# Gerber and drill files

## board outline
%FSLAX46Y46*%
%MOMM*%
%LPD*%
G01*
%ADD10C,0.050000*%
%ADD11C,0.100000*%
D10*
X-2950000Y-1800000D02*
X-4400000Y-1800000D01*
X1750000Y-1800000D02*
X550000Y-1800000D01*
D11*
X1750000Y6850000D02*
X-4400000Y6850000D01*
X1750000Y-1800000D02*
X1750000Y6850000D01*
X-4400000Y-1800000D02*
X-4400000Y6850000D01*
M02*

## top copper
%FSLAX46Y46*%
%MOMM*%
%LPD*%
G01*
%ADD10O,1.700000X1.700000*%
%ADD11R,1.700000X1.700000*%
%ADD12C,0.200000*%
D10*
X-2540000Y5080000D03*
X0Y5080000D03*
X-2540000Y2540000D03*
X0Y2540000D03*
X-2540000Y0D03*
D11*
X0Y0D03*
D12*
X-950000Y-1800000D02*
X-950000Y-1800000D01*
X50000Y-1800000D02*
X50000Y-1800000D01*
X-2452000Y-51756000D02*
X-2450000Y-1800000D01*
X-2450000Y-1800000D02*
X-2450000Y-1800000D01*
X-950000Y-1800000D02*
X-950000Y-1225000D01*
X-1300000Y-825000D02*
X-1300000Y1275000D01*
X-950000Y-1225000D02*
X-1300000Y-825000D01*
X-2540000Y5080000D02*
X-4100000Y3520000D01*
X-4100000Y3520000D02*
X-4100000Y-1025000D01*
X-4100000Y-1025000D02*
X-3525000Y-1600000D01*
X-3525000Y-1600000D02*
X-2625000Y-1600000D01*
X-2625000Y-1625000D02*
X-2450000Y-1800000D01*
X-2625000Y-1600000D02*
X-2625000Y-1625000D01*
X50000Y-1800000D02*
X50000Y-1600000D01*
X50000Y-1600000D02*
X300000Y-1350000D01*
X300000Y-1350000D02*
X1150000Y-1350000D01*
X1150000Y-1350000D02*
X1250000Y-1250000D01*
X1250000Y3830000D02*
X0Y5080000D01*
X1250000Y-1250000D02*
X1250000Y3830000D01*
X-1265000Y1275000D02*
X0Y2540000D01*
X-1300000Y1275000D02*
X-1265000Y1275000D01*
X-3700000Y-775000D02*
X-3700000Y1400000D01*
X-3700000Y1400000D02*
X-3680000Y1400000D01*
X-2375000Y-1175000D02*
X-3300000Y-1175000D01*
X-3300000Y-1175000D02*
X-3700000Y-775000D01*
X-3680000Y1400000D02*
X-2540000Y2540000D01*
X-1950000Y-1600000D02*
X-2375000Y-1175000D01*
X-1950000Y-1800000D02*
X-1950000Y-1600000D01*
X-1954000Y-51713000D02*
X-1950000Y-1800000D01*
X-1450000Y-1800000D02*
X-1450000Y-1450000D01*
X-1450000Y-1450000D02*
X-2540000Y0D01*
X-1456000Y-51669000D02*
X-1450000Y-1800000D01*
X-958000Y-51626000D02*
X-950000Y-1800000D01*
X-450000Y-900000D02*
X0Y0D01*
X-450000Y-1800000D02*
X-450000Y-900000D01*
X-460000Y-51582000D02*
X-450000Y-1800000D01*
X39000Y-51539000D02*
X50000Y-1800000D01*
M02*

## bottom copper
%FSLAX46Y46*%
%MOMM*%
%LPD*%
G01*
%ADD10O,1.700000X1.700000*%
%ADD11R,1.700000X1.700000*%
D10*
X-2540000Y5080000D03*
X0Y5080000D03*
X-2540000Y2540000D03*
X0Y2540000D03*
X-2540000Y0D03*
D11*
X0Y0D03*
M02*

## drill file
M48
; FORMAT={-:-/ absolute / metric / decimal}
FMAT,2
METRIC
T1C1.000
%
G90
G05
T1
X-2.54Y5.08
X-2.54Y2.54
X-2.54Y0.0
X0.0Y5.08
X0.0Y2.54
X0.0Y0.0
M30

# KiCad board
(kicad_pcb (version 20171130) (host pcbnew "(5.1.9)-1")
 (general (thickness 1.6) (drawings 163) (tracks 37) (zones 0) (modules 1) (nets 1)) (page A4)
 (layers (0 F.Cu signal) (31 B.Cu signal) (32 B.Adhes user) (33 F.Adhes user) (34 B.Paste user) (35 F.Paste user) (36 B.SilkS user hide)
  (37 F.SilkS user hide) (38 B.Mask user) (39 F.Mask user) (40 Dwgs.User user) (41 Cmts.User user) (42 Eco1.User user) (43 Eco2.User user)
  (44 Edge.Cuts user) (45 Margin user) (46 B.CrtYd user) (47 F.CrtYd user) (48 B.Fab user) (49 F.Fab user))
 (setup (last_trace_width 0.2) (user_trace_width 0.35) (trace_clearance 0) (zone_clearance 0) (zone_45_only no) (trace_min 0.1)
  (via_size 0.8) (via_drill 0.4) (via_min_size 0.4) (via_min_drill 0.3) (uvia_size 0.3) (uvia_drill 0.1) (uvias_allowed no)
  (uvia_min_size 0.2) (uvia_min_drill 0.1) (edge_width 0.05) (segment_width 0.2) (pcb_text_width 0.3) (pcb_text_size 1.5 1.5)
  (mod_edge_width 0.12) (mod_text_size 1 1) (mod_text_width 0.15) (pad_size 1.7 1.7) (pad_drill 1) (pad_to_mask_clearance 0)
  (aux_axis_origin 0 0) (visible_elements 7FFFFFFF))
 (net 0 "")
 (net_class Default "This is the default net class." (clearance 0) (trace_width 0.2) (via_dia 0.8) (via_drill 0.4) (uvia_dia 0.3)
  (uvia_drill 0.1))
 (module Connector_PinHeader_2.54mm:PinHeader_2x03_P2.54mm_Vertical (layer F.Cu) (at 0 0 180)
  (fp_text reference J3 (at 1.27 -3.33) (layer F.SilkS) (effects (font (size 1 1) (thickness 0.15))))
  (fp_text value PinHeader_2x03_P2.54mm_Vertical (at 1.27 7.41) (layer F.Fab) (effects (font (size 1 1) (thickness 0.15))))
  (pad 6 thru_hole oval (at 2.54 5.08) (size 1.7 1.7) (drill 1) (layers *.Cu *.Mask))
  (pad 5 thru_hole oval (at 0 5.08) (size 1.7 1.7) (drill 1) (layers *.Cu *.Mask))
  (pad 4 thru_hole oval (at 2.54 2.54) (size 1.7 1.7) (drill 1) (layers *.Cu *.Mask))
  (pad 3 thru_hole oval (at 0 2.54) (size 1.7 1.7) (drill 1) (layers *.Cu *.Mask))
  (pad 2 thru_hole oval (at 2.54 0) (size 1.7 1.7) (drill 1) (layers *.Cu *.Mask))
  (pad 1 thru_hole rect (at 0 0) (size 1.7 1.7) (drill 1) (layers *.Cu *.Mask)))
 (gr_line (start -2.95 1.8) (end -4.4 1.8) (layer Edge.Cuts) (width 0.05))
 (gr_line (start 1.75 1.8) (end 0.55 1.8) (layer Edge.Cuts) (width 0.05))
 (gr_line (start 1.75 -6.85) (end -4.4 -6.85) (layer Edge.Cuts) (width 0.1))
 (gr_line (start 1.75 1.8) (end 1.75 -6.85) (layer Edge.Cuts) (width 0.1))
 (gr_line (start -4.4 1.8) (end -4.4 -6.85) (layer Edge.Cuts) (width 0.1))
 (segment (start -0.95 1.8) (end -0.95 1.8) (width 0.2) (layer F.Cu) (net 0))
 (segment (start 0.05 1.8) (end 0.05 1.8) (width 0.2) (layer F.Cu) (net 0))
 (segment (start -2.452 51.756) (end -2.45 1.8) (width 0.2) (layer F.Cu) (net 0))
 (segment (start -2.45 1.8) (end -2.45 1.8) (width 0.2) (layer F.Cu) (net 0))
 (segment (start -0.95 1.8) (end -0.95 1.225) (width 0.2) (layer F.Cu) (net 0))
 (segment (start -1.3 0.825) (end -1.3 -1.275) (width 0.2) (layer F.Cu) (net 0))
 (segment (start -0.95 1.225) (end -1.3 0.825) (width 0.2) (layer F.Cu) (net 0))
 (segment (start -2.54 -5.08) (end -4.1 -3.52) (width 0.2) (layer F.Cu) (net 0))
 (segment (start -4.1 -3.52) (end -4.1 1.025) (width 0.2) (layer F.Cu) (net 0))
 (segment (start -4.1 1.025) (end -3.525 1.6) (width 0.2) (layer F.Cu) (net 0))
 (segment (start -3.525 1.6) (end -2.625 1.6) (width 0.2) (layer F.Cu) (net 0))
 (segment (start -2.625 1.625) (end -2.45 1.8) (width 0.2) (layer F.Cu) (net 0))
 (segment (start -2.625 1.6) (end -2.625 1.625) (width 0.2) (layer F.Cu) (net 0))
 (segment (start 0.05 1.8) (end 0.05 1.6) (width 0.2) (layer F.Cu) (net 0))
 (segment (start 0.05 1.6) (end 0.3 1.35) (width 0.2) (layer F.Cu) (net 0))
 (segment (start 0.3 1.35) (end 1.15 1.35) (width 0.2) (layer F.Cu) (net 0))
 (segment (start 1.15 1.35) (end 1.25 1.25) (width 0.2) (layer F.Cu) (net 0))
 (segment (start 1.25 -3.83) (end 0 -5.08) (width 0.2) (layer F.Cu) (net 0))
 (segment (start 1.25 1.25) (end 1.25 -3.83) (width 0.2) (layer F.Cu) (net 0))
 (segment (start -1.265 -1.275) (end 0 -2.54) (width 0.2) (layer F.Cu) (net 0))
 (segment (start -1.3 -1.275) (end -1.265 -1.275) (width 0.2) (layer F.Cu) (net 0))
 (segment (start -3.7 0.775) (end -3.7 -1.4) (width 0.2) (layer F.Cu) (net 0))
 (segment (start -3.7 -1.4) (end -3.68 -1.4) (width 0.2) (layer F.Cu) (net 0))
 (segment (start -2.375 1.175) (end -3.3 1.175) (width 0.2) (layer F.Cu) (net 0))
 (segment (start -3.3 1.175) (end -3.7 0.775) (width 0.2) (layer F.Cu) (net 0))
 (segment (start -3.68 -1.4) (end -2.54 -2.54) (width 0.2) (layer F.Cu) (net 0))
 (segment (start -1.95 1.6) (end -2.375 1.175) (width 0.2) (layer F.Cu) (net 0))
 (segment (start -1.95 1.8) (end -1.95 1.6) (width 0.2) (layer F.Cu) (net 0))
 (segment (start -1.954 51.713) (end -1.95 1.8) (width 0.2) (layer F.Cu) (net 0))
 (segment (start -1.45 1.8) (end -1.45 1.45) (width 0.2) (layer F.Cu) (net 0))
 (segment (start -1.45 1.45) (end -2.54 0) (width 0.2) (layer F.Cu) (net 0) (status 800000))
 (segment (start -1.456 51.669) (end -1.45 1.8) (width 0.2) (layer F.Cu) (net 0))
 (segment (start -0.958 51.626) (end -0.95 1.8) (width 0.2) (layer F.Cu) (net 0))
 (segment (start -0.45 0.9) (end 0 0) (width 0.2) (layer F.Cu) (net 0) (status 800000))
 (segment (start -0.45 1.8) (end -0.45 0.9) (width 0.2) (layer F.Cu) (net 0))
 (segment (start -0.46 51.582) (end -0.45 1.8) (width 0.2) (layer F.Cu) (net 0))
 (segment (start 0.039 51.539) (end 0.05 1.8) (width 0.2) (layer F.Cu) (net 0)))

